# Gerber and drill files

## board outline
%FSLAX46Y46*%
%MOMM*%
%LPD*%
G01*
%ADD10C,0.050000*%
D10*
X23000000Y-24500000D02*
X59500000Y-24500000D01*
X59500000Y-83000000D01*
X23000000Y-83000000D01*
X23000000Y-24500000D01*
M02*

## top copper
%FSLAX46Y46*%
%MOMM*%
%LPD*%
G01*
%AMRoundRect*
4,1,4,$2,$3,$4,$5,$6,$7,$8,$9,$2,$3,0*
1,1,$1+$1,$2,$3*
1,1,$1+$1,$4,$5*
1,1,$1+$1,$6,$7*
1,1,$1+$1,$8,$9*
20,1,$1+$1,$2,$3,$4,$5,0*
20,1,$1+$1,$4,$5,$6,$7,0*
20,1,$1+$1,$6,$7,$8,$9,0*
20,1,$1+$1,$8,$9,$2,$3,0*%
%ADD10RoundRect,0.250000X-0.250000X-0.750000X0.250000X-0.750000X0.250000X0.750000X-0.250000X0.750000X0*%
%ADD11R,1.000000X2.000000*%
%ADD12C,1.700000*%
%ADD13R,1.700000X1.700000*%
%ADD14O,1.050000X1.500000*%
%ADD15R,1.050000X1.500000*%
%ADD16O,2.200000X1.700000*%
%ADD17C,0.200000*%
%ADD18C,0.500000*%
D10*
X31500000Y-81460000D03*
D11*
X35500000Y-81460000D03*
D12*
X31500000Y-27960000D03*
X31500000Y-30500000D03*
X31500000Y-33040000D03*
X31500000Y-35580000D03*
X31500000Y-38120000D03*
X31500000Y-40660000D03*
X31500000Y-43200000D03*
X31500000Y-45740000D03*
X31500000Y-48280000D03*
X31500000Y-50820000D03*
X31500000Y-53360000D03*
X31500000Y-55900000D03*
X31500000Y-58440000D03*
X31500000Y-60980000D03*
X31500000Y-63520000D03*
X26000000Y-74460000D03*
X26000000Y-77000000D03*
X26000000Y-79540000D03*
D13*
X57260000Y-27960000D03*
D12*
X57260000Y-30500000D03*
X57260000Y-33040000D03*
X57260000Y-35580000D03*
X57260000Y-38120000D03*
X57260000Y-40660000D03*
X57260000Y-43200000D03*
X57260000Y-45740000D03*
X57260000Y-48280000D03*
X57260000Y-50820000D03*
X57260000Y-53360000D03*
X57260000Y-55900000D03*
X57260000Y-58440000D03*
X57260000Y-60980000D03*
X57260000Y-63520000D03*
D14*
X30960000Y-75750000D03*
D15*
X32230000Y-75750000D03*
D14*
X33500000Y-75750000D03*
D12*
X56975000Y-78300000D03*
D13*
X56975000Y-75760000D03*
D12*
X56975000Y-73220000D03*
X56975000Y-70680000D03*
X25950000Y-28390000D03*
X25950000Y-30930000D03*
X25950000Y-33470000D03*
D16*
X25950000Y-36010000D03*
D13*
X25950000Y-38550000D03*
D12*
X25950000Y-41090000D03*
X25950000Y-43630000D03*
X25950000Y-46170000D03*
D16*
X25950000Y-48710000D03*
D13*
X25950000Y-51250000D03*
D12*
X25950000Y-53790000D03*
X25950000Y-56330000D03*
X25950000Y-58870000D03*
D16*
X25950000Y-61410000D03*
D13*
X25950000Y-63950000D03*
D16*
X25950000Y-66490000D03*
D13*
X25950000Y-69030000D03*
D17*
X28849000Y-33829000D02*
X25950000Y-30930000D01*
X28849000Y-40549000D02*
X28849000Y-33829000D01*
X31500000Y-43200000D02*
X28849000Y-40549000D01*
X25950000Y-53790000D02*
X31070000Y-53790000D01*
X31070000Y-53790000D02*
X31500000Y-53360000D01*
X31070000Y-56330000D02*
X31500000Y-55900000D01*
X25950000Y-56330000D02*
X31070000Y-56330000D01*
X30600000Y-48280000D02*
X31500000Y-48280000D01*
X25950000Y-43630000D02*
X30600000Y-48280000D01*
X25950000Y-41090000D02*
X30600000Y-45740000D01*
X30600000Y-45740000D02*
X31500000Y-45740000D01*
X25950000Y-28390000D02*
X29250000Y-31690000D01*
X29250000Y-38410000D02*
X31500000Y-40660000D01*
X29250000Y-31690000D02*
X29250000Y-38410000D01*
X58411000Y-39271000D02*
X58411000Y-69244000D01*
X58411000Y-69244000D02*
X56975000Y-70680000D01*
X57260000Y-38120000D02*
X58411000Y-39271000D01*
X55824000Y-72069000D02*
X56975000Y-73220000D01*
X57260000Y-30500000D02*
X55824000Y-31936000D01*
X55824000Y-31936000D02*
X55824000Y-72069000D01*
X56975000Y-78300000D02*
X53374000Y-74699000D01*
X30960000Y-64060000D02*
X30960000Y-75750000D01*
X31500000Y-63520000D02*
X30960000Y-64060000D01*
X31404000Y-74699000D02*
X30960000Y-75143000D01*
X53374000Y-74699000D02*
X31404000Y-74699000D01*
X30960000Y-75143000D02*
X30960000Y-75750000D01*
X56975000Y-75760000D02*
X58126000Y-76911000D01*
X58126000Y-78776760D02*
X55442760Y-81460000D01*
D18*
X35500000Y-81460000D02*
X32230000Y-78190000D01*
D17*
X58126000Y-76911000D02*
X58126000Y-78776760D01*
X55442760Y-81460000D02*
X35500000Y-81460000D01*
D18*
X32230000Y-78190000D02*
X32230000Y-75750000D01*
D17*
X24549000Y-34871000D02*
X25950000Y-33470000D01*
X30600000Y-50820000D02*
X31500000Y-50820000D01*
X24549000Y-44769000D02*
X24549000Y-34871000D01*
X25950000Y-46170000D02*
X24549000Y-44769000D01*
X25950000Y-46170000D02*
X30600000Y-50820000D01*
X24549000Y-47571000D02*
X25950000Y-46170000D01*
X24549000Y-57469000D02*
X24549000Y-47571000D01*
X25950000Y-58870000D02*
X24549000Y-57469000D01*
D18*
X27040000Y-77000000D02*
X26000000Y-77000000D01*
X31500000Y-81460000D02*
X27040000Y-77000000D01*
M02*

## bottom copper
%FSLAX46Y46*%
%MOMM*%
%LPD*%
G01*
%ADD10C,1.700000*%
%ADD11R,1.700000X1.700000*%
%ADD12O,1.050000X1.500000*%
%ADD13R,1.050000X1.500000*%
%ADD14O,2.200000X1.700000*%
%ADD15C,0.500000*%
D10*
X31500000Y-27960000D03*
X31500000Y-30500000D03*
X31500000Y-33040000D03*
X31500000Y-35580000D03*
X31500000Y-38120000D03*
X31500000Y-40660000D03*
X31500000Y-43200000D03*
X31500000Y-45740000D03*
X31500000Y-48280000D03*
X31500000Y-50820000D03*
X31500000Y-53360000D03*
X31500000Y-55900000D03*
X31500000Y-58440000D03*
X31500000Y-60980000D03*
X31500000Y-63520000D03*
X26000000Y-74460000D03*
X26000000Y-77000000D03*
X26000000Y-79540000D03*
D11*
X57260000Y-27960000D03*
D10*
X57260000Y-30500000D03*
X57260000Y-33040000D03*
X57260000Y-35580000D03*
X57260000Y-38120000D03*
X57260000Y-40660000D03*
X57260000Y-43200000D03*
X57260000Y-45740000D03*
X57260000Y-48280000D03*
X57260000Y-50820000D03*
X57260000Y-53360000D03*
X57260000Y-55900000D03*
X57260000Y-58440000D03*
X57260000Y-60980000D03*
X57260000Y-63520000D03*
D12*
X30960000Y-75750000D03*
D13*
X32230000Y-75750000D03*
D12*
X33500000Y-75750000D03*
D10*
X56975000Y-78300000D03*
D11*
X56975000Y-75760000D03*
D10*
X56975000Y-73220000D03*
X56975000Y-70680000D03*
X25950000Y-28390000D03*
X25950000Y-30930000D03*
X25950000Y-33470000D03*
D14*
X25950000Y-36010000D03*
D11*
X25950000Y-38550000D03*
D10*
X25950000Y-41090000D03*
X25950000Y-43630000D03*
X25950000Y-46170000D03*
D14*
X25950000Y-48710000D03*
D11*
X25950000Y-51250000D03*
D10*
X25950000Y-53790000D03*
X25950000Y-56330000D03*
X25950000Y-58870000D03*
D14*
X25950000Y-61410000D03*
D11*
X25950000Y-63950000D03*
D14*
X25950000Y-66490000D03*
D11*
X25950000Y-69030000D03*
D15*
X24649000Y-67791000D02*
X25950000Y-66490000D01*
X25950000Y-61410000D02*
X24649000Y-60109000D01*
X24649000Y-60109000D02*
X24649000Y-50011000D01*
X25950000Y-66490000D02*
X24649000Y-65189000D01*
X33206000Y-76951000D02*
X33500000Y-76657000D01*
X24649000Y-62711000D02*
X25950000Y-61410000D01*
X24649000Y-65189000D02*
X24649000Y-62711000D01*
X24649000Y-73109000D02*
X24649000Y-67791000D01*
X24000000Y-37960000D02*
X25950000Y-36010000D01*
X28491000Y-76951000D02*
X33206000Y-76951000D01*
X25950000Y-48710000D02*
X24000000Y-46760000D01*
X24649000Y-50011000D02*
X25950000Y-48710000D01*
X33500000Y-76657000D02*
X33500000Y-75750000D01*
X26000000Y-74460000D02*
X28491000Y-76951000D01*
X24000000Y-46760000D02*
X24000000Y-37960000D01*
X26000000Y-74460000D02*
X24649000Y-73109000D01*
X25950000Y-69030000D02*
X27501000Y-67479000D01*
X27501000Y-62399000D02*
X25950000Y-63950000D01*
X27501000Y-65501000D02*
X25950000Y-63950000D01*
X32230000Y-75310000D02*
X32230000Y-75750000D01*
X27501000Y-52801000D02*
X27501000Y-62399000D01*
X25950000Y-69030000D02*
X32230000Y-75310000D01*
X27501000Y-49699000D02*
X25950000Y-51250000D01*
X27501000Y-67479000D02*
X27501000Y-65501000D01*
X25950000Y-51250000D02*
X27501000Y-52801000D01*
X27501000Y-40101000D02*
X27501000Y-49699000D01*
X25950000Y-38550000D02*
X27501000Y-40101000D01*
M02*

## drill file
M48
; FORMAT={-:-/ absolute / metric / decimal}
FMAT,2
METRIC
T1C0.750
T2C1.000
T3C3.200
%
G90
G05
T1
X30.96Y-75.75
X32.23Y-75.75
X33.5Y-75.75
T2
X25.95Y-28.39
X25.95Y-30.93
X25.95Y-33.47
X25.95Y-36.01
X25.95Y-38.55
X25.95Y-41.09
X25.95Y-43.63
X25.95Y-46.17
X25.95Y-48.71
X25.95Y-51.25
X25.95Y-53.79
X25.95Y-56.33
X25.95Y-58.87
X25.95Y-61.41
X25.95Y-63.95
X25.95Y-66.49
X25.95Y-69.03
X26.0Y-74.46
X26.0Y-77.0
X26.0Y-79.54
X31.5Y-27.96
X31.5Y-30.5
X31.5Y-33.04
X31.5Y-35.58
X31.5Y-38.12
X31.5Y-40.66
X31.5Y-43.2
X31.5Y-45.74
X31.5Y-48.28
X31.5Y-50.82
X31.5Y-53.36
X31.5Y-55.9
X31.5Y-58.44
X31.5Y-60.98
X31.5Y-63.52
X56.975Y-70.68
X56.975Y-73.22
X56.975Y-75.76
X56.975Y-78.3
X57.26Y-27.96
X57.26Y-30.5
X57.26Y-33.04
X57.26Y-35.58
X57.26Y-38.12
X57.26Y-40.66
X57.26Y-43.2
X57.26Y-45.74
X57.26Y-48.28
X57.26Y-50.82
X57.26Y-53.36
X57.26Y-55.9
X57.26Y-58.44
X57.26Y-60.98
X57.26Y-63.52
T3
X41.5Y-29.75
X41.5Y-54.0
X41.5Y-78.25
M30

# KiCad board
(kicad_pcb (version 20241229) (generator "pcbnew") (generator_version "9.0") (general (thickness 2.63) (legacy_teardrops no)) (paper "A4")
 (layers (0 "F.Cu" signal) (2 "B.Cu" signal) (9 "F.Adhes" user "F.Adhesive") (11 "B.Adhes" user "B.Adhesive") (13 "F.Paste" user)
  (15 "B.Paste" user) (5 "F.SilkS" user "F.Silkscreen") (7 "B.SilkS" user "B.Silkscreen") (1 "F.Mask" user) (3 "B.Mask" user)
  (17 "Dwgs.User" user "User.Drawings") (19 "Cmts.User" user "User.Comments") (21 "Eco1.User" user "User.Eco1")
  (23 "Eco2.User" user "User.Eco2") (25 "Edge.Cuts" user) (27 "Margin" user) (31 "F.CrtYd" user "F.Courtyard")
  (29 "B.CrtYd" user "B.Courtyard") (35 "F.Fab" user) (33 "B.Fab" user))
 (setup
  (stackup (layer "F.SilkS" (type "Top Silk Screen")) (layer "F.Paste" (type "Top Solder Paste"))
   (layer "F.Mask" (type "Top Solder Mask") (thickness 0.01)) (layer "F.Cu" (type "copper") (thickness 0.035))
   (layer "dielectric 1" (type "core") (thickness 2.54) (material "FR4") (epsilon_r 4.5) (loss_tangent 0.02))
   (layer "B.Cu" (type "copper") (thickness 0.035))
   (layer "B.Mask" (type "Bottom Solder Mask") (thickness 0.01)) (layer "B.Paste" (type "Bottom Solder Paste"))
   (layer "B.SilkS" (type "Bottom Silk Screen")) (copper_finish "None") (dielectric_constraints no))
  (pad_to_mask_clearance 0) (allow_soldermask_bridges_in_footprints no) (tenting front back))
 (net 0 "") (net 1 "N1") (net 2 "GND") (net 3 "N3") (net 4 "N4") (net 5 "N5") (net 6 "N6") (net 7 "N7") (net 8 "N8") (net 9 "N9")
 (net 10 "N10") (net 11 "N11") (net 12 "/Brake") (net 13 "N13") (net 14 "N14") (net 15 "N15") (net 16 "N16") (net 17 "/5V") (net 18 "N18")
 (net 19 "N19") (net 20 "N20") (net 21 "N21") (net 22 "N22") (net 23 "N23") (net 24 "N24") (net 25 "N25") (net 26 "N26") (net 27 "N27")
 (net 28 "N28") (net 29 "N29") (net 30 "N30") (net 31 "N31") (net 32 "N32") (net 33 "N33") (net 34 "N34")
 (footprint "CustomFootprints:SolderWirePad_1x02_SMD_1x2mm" (layer "F.Cu") (at 33.5 81.46)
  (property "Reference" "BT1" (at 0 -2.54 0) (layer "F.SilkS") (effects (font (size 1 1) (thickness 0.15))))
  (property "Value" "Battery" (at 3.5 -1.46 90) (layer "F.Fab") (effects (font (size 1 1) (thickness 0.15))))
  (pad "1" smd roundrect (at -2 0) (size 1 2) (layers "F.Cu" "F.Mask" "F.Paste") (roundrect_rratio 0.25) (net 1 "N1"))
  (pad "2" smd rect (at 2 0) (size 1 2) (layers "F.Cu" "F.Mask" "F.Paste") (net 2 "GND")))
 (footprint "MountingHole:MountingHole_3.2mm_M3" (layer "F.Cu") (at 41.5 78.25)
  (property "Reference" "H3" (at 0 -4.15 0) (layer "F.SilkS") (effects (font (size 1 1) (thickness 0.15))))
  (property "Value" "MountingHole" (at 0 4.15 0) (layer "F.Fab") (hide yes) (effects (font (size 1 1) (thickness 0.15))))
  (pad "" np_thru_hole circle (at 0 0) (size 3.2 3.2) (drill 3.2) (layers "*.Cu" "*.Mask")))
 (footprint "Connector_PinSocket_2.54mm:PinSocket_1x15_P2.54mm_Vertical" (layer "F.Cu") (at 31.5 27.96)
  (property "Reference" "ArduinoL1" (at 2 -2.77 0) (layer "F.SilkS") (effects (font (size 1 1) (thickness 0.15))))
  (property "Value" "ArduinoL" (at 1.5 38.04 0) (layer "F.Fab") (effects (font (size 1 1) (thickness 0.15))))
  (pad "1" thru_hole circle (at 0 0) (size 1.7 1.7) (drill 1) (layers "*.Cu" "*.Mask") (remove_unused_layers no) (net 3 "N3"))
  (pad "2" thru_hole circle (at 0 2.54) (size 1.7 1.7) (drill 1) (layers "*.Cu" "*.Mask") (remove_unused_layers no) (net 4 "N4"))
  (pad "3" thru_hole circle (at 0 5.08) (size 1.7 1.7) (drill 1) (layers "*.Cu" "*.Mask") (remove_unused_layers no) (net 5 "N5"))
  (pad "4" thru_hole circle (at 0 7.62) (size 1.7 1.7) (drill 1) (layers "*.Cu" "*.Mask") (remove_unused_layers no) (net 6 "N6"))
  (pad "5" thru_hole circle (at 0 10.16) (size 1.7 1.7) (drill 1) (layers "*.Cu" "*.Mask") (remove_unused_layers no) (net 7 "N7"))
  (pad "6" thru_hole circle (at 0 12.7) (size 1.7 1.7) (drill 1) (layers "*.Cu" "*.Mask") (remove_unused_layers no) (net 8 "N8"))
  (pad "7" thru_hole circle (at 0 15.24) (size 1.7 1.7) (drill 1) (layers "*.Cu" "*.Mask") (remove_unused_layers no) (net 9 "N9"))
  (pad "8" thru_hole circle (at 0 17.78) (size 1.7 1.7) (drill 1) (layers "*.Cu" "*.Mask") (remove_unused_layers no) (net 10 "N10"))
  (pad "9" thru_hole circle (at 0 20.32) (size 1.7 1.7) (drill 1) (layers "*.Cu" "*.Mask") (remove_unused_layers no) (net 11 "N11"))
  (pad "10" thru_hole circle (at 0 22.86) (size 1.7 1.7) (drill 1) (layers "*.Cu" "*.Mask") (remove_unused_layers no) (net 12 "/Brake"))
  (pad "11" thru_hole circle (at 0 25.4) (size 1.7 1.7) (drill 1) (layers "*.Cu" "*.Mask") (remove_unused_layers no) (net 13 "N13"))
  (pad "12" thru_hole circle (at 0 27.94) (size 1.7 1.7) (drill 1) (layers "*.Cu" "*.Mask") (remove_unused_layers no) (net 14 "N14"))
  (pad "13" thru_hole circle (at 0 30.48) (size 1.7 1.7) (drill 1) (layers "*.Cu" "*.Mask") (remove_unused_layers no) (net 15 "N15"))
  (pad "14" thru_hole circle (at 0 33.02) (size 1.7 1.7) (drill 1) (layers "*.Cu" "*.Mask") (remove_unused_layers no) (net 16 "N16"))
  (pad "15" thru_hole circle (at 0 35.56) (size 1.7 1.7) (drill 1) (layers "*.Cu" "*.Mask") (remove_unused_layers no) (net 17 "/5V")))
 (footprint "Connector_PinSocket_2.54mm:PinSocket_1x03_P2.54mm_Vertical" (layer "F.Cu") (at 26 74.46)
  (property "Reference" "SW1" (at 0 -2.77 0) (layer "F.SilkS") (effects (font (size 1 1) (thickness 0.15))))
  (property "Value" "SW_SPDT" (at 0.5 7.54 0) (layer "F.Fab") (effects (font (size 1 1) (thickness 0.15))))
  (pad "1" thru_hole circle (at 0 0) (size 1.7 1.7) (drill 1) (layers "*.Cu" "*.Mask") (remove_unused_layers no) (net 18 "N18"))
  (pad "2" thru_hole circle (at 0 2.54) (size 1.7 1.7) (drill 1) (layers "*.Cu" "*.Mask") (remove_unused_layers no) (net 1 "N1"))
  (pad "3" thru_hole circle (at 0 5.08) (size 1.7 1.7) (drill 1) (layers "*.Cu" "*.Mask") (remove_unused_layers no) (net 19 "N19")))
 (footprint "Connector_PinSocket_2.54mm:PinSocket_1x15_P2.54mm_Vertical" (layer "F.Cu") (at 57.26 27.96)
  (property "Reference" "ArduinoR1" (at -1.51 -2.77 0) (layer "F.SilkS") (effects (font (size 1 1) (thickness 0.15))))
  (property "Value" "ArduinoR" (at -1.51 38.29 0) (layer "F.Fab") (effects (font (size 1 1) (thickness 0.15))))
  (pad "1" thru_hole rect (at 0 0) (size 1.7 1.7) (drill 1) (layers "*.Cu" "*.Mask") (remove_unused_layers no) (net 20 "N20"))
  (pad "2" thru_hole circle (at 0 2.54) (size 1.7 1.7) (drill 1) (layers "*.Cu" "*.Mask") (remove_unused_layers no) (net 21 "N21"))
  (pad "3" thru_hole circle (at 0 5.08) (size 1.7 1.7) (drill 1) (layers "*.Cu" "*.Mask") (remove_unused_layers no) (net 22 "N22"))
  (pad "4" thru_hole circle (at 0 7.62) (size 1.7 1.7) (drill 1) (layers "*.Cu" "*.Mask") (remove_unused_layers no) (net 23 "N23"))
  (pad "5" thru_hole circle (at 0 10.16) (size 1.7 1.7) (drill 1) (layers "*.Cu" "*.Mask") (remove_unused_layers no) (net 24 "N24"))
  (pad "6" thru_hole circle (at 0 12.7) (size 1.7 1.7) (drill 1) (layers "*.Cu" "*.Mask") (remove_unused_layers no) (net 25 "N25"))
  (pad "7" thru_hole circle (at 0 15.24) (size 1.7 1.7) (drill 1) (layers "*.Cu" "*.Mask") (remove_unused_layers no) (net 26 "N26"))
  (pad "8" thru_hole circle (at 0 17.78) (size 1.7 1.7) (drill 1) (layers "*.Cu" "*.Mask") (remove_unused_layers no) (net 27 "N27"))
  (pad "9" thru_hole circle (at 0 20.32) (size 1.7 1.7) (drill 1) (layers "*.Cu" "*.Mask") (remove_unused_layers no) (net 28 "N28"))
  (pad "10" thru_hole circle (at 0 22.86) (size 1.7 1.7) (drill 1) (layers "*.Cu" "*.Mask") (remove_unused_layers no) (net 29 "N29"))
  (pad "11" thru_hole circle (at 0 25.4) (size 1.7 1.7) (drill 1) (layers "*.Cu" "*.Mask") (remove_unused_layers no) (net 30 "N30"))
  (pad "12" thru_hole circle (at 0 27.94) (size 1.7 1.7) (drill 1) (layers "*.Cu" "*.Mask") (remove_unused_layers no) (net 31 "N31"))
  (pad "13" thru_hole circle (at 0 30.48) (size 1.7 1.7) (drill 1) (layers "*.Cu" "*.Mask") (remove_unused_layers no) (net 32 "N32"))
  (pad "14" thru_hole circle (at 0 33.02) (size 1.7 1.7) (drill 1) (layers "*.Cu" "*.Mask") (remove_unused_layers no) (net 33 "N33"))
  (pad "15" thru_hole circle (at 0 35.56) (size 1.7 1.7) (drill 1) (layers "*.Cu" "*.Mask") (remove_unused_layers no) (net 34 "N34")))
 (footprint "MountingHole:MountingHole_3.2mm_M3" (layer "F.Cu") (at 41.5 54)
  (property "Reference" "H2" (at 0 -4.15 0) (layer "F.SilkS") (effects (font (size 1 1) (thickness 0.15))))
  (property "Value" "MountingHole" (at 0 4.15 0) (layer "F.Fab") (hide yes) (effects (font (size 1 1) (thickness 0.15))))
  (pad "" np_thru_hole circle (at 0 0) (size 3.2 3.2) (drill 3.2) (layers "*.Cu" "*.Mask")))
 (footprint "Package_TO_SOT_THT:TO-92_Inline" (layer "F.Cu") (at 30.96 75.75)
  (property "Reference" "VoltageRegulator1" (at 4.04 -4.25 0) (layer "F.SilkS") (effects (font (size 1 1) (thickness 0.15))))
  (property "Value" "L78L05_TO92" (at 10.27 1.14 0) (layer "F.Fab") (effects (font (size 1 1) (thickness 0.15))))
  (pad "1" thru_hole oval (at 0 0) (size 1.05 1.5) (drill 0.75) (layers "*.Cu" "*.Mask") (remove_unused_layers no) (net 17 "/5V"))
  (pad "2" thru_hole rect (at 1.27 0) (size 1.05 1.5) (drill 0.75) (layers "*.Cu" "*.Mask") (remove_unused_layers no) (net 2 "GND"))
  (pad "3" thru_hole oval (at 2.54 0) (size 1.05 1.5) (drill 0.75) (layers "*.Cu" "*.Mask") (remove_unused_layers no) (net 18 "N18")))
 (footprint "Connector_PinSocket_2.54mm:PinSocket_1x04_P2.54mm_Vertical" (layer "F.Cu") (at 56.975 78.3 180)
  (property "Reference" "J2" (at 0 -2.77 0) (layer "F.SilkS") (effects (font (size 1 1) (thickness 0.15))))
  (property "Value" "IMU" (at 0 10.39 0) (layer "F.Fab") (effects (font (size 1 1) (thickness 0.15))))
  (pad "1" thru_hole circle (at 0 0 180) (size 1.7 1.7) (drill 1) (layers "*.Cu" "*.Mask") (remove_unused_layers no) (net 17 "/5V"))
  (pad "2" thru_hole rect (at 0 2.54 180) (size 1.7 1.7) (drill 1) (layers "*.Cu" "*.Mask") (remove_unused_layers no) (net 2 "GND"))
  (pad "3" thru_hole circle (at 0 5.08 180) (size 1.7 1.7) (drill 1) (layers "*.Cu" "*.Mask") (remove_unused_layers no) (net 21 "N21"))
  (pad "4" thru_hole circle (at 0 7.62 180) (size 1.7 1.7) (drill 1) (layers "*.Cu" "*.Mask") (remove_unused_layers no) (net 24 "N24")))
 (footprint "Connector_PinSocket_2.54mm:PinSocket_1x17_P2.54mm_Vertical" (layer "F.Cu") (at 25.95 28.39)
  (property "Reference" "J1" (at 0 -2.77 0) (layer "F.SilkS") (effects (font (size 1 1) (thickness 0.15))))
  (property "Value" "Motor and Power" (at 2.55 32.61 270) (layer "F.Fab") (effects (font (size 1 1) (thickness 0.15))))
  (pad "1" thru_hole circle (at 0 0) (size 1.7 1.7) (drill 1) (layers "*.Cu" "*.Mask") (remove_unused_layers no) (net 8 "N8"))
  (pad "2" thru_hole circle (at 0 2.54) (size 1.7 1.7) (drill 1) (layers "*.Cu" "*.Mask") (remove_unused_layers no) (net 9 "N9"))
  (pad "3" thru_hole circle (at 0 5.08) (size 1.7 1.7) (drill 1) (layers "*.Cu" "*.Mask") (remove_unused_layers no) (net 12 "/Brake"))
  (pad "4" thru_hole oval (at 0 7.62) (size 2.2 1.7) (drill 1) (layers "*.Cu" "*.Mask") (remove_unused_layers no) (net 18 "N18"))
  (pad "5" thru_hole rect (at 0 10.16) (size 1.7 1.7) (drill 1) (layers "*.Cu" "*.Mask") (remove_unused_layers no) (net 2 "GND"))
  (pad "6" thru_hole circle (at 0 12.7) (size 1.7 1.7) (drill 1) (layers "*.Cu" "*.Mask") (remove_unused_layers no) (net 10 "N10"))
  (pad "7" thru_hole circle (at 0 15.24) (size 1.7 1.7) (drill 1) (layers "*.Cu" "*.Mask") (remove_unused_layers no) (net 11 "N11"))
  (pad "8" thru_hole circle (at 0 17.78) (size 1.7 1.7) (drill 1) (layers "*.Cu" "*.Mask") (remove_unused_layers no) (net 12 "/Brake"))
  (pad "9" thru_hole oval (at 0 20.32) (size 2.2 1.7) (drill 1) (layers "*.Cu" "*.Mask") (remove_unused_layers no) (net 18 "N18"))
  (pad "10" thru_hole rect (at 0 22.86) (size 1.7 1.7) (drill 1) (layers "*.Cu" "*.Mask") (remove_unused_layers no) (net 2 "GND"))
  (pad "11" thru_hole circle (at 0 25.4) (size 1.7 1.7) (drill 1) (layers "*.Cu" "*.Mask") (remove_unused_layers no) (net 13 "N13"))
  (pad "12" thru_hole circle (at 0 27.94) (size 1.7 1.7) (drill 1) (layers "*.Cu" "*.Mask") (remove_unused_layers no) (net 14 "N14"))
  (pad "13" thru_hole circle (at 0 30.48) (size 1.7 1.7) (drill 1) (layers "*.Cu" "*.Mask") (remove_unused_layers no) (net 12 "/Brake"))
  (pad "14" thru_hole oval (at 0 33.02) (size 2.2 1.7) (drill 1) (layers "*.Cu" "*.Mask") (remove_unused_layers no) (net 18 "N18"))
  (pad "15" thru_hole rect (at 0 35.56) (size 1.7 1.7) (drill 1) (layers "*.Cu" "*.Mask") (remove_unused_layers no) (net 2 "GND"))
  (pad "16" thru_hole oval (at 0 38.1) (size 2.2 1.7) (drill 1) (layers "*.Cu" "*.Mask") (remove_unused_layers no) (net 18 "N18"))
  (pad "17" thru_hole rect (at 0 40.64) (size 1.7 1.7) (drill 1) (layers "*.Cu" "*.Mask") (remove_unused_layers no) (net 2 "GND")))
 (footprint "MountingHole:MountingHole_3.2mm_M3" (layer "F.Cu") (at 41.5 29.75)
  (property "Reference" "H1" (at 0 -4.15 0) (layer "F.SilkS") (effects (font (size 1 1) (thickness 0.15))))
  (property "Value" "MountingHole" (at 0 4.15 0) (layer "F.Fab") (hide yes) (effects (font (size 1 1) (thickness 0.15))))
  (pad "" np_thru_hole circle (at 0 0) (size 3.2 3.2) (drill 3.2) (layers "*.Cu" "*.Mask")))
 (gr_rect (start 23 24.5) (end 59.5 83) (stroke (width 0.05) (type solid)) (fill no) (layer "Edge.Cuts"))
 (segment (start 28.849 33.829) (end 25.95 30.93) (width 0.2) (layer "F.Cu") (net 9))
 (segment (start 28.849 40.549) (end 28.849 33.829) (width 0.2) (layer "F.Cu") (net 9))
 (segment (start 31.5 43.2) (end 28.849 40.549) (width 0.2) (layer "F.Cu") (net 9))
 (segment (start 25.95 53.79) (end 31.07 53.79) (width 0.2) (layer "F.Cu") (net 13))
 (segment (start 31.07 53.79) (end 31.5 53.36) (width 0.2) (layer "F.Cu") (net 13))
 (segment (start 31.07 56.33) (end 31.5 55.9) (width 0.2) (layer "F.Cu") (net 14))
 (segment (start 25.95 56.33) (end 31.07 56.33) (width 0.2) (layer "F.Cu") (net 14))
 (segment (start 30.6 48.28) (end 31.5 48.28) (width 0.2) (layer "F.Cu") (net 11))
 (segment (start 25.95 43.63) (end 30.6 48.28) (width 0.2) (layer "F.Cu") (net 11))
 (segment (start 25.95 41.09) (end 30.6 45.74) (width 0.2) (layer "F.Cu") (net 10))
 (segment (start 30.6 45.74) (end 31.5 45.74) (width 0.2) (layer "F.Cu") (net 10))
 (segment (start 25.95 28.39) (end 29.25 31.69) (width 0.2) (layer "F.Cu") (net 8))
 (segment (start 29.25 38.41) (end 31.5 40.66) (width 0.2) (layer "F.Cu") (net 8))
 (segment (start 29.25 31.69) (end 29.25 38.41) (width 0.2) (layer "F.Cu") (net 8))
 (segment (start 58.411 39.271) (end 58.411 69.244) (width 0.2) (layer "F.Cu") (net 24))
 (segment (start 58.411 69.244) (end 56.975 70.68) (width 0.2) (layer "F.Cu") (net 24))
 (segment (start 57.26 38.12) (end 58.411 39.271) (width 0.2) (layer "F.Cu") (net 24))
 (segment (start 55.824 72.069) (end 56.975 73.22) (width 0.2) (layer "F.Cu") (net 21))
 (segment (start 57.26 30.5) (end 55.824 31.936) (width 0.2) (layer "F.Cu") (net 21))
 (segment (start 55.824 31.936) (end 55.824 72.069) (width 0.2) (layer "F.Cu") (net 21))
 (segment (start 24.649 67.791) (end 25.95 66.49) (width 0.5) (layer "B.Cu") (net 18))
 (segment (start 25.95 61.41) (end 24.649 60.109) (width 0.5) (layer "B.Cu") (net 18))
 (segment (start 24.649 60.109) (end 24.649 50.011) (width 0.5) (layer "B.Cu") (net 18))
 (segment (start 25.95 66.49) (end 24.649 65.189) (width 0.5) (layer "B.Cu") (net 18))
 (segment (start 33.206 76.951) (end 33.5 76.657) (width 0.5) (layer "B.Cu") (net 18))
 (segment (start 24.649 62.711) (end 25.95 61.41) (width 0.5) (layer "B.Cu") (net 18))
 (segment (start 24.649 65.189) (end 24.649 62.711) (width 0.5) (layer "B.Cu") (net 18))
 (segment (start 24.649 73.109) (end 24.649 67.791) (width 0.5) (layer "B.Cu") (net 18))
 (segment (start 24 37.96) (end 25.95 36.01) (width 0.5) (layer "B.Cu") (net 18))
 (segment (start 28.491 76.951) (end 33.206 76.951) (width 0.5) (layer "B.Cu") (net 18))
 (segment (start 25.95 48.71) (end 24 46.76) (width 0.5) (layer "B.Cu") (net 18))
 (segment (start 24.649 50.011) (end 25.95 48.71) (width 0.5) (layer "B.Cu") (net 18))
 (segment (start 33.5 76.657) (end 33.5 75.75) (width 0.5) (layer "B.Cu") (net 18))
 (segment (start 26 74.46) (end 28.491 76.951) (width 0.5) (layer "B.Cu") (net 18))
 (segment (start 24 46.76) (end 24 37.96) (width 0.5) (layer "B.Cu") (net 18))
 (segment (start 26 74.46) (end 24.649 73.109) (width 0.5) (layer "B.Cu") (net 18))
 (segment (start 56.975 78.3) (end 53.374 74.699) (width 0.2) (layer "F.Cu") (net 17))
 (segment (start 30.96 64.06) (end 30.96 75.75) (width 0.2) (layer "F.Cu") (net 17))
 (segment (start 31.5 63.52) (end 30.96 64.06) (width 0.2) (layer "F.Cu") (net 17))
 (segment (start 31.404 74.699) (end 30.96 75.143) (width 0.2) (layer "F.Cu") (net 17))
 (segment (start 53.374 74.699) (end 31.404 74.699) (width 0.2) (layer "F.Cu") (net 17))
 (segment (start 30.96 75.143) (end 30.96 75.75) (width 0.2) (layer "F.Cu") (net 17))
 (segment (start 56.975 75.76) (end 58.126 76.911) (width 0.2) (layer "F.Cu") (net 2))
 (segment (start 58.126 78.77676) (end 55.44276 81.46) (width 0.2) (layer "F.Cu") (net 2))
 (segment (start 35.5 81.46) (end 32.23 78.19) (width 0.5) (layer "F.Cu") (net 2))
 (segment (start 58.126 76.911) (end 58.126 78.77676) (width 0.2) (layer "F.Cu") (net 2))
 (segment (start 55.44276 81.46) (end 35.5 81.46) (width 0.2) (layer "F.Cu") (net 2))
 (segment (start 32.23 78.19) (end 32.23 75.75) (width 0.5) (layer "F.Cu") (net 2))
 (segment (start 25.95 69.03) (end 27.501 67.479) (width 0.5) (layer "B.Cu") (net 2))
 (segment (start 27.501 62.399) (end 25.95 63.95) (width 0.5) (layer "B.Cu") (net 2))
 (segment (start 27.501 65.501) (end 25.95 63.95) (width 0.5) (layer "B.Cu") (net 2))
 (segment (start 32.23 75.31) (end 32.23 75.75) (width 0.5) (layer "B.Cu") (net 2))
 (segment (start 27.501 52.801) (end 27.501 62.399) (width 0.5) (layer "B.Cu") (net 2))
 (segment (start 25.95 69.03) (end 32.23 75.31) (width 0.5) (layer "B.Cu") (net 2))
 (segment (start 27.501 49.699) (end 25.95 51.25) (width 0.5) (layer "B.Cu") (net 2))
 (segment (start 27.501 67.479) (end 27.501 65.501) (width 0.5) (layer "B.Cu") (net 2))
 (segment (start 25.95 51.25) (end 27.501 52.801) (width 0.5) (layer "B.Cu") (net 2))
 (segment (start 27.501 40.101) (end 27.501 49.699) (width 0.5) (layer "B.Cu") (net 2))
 (segment (start 25.95 38.55) (end 27.501 40.101) (width 0.5) (layer "B.Cu") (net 2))
 (segment (start 24.549 34.871) (end 25.95 33.47) (width 0.2) (layer "F.Cu") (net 12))
 (segment (start 30.6 50.82) (end 31.5 50.82) (width 0.2) (layer "F.Cu") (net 12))
 (segment (start 24.549 44.769) (end 24.549 34.871) (width 0.2) (layer "F.Cu") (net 12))
 (segment (start 25.95 46.17) (end 24.549 44.769) (width 0.2) (layer "F.Cu") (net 12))
 (segment (start 25.95 46.17) (end 30.6 50.82) (width 0.2) (layer "F.Cu") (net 12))
 (segment (start 24.549 47.571) (end 25.95 46.17) (width 0.2) (layer "F.Cu") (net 12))
 (segment (start 24.549 57.469) (end 24.549 47.571) (width 0.2) (layer "F.Cu") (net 12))
 (segment (start 25.95 58.87) (end 24.549 57.469) (width 0.2) (layer "F.Cu") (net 12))
 (segment (start 27.04 77) (end 26 77) (width 0.5) (layer "F.Cu") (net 1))
 (segment (start 31.5 81.46) (end 27.04 77) (width 0.5) (layer "F.Cu") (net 1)))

